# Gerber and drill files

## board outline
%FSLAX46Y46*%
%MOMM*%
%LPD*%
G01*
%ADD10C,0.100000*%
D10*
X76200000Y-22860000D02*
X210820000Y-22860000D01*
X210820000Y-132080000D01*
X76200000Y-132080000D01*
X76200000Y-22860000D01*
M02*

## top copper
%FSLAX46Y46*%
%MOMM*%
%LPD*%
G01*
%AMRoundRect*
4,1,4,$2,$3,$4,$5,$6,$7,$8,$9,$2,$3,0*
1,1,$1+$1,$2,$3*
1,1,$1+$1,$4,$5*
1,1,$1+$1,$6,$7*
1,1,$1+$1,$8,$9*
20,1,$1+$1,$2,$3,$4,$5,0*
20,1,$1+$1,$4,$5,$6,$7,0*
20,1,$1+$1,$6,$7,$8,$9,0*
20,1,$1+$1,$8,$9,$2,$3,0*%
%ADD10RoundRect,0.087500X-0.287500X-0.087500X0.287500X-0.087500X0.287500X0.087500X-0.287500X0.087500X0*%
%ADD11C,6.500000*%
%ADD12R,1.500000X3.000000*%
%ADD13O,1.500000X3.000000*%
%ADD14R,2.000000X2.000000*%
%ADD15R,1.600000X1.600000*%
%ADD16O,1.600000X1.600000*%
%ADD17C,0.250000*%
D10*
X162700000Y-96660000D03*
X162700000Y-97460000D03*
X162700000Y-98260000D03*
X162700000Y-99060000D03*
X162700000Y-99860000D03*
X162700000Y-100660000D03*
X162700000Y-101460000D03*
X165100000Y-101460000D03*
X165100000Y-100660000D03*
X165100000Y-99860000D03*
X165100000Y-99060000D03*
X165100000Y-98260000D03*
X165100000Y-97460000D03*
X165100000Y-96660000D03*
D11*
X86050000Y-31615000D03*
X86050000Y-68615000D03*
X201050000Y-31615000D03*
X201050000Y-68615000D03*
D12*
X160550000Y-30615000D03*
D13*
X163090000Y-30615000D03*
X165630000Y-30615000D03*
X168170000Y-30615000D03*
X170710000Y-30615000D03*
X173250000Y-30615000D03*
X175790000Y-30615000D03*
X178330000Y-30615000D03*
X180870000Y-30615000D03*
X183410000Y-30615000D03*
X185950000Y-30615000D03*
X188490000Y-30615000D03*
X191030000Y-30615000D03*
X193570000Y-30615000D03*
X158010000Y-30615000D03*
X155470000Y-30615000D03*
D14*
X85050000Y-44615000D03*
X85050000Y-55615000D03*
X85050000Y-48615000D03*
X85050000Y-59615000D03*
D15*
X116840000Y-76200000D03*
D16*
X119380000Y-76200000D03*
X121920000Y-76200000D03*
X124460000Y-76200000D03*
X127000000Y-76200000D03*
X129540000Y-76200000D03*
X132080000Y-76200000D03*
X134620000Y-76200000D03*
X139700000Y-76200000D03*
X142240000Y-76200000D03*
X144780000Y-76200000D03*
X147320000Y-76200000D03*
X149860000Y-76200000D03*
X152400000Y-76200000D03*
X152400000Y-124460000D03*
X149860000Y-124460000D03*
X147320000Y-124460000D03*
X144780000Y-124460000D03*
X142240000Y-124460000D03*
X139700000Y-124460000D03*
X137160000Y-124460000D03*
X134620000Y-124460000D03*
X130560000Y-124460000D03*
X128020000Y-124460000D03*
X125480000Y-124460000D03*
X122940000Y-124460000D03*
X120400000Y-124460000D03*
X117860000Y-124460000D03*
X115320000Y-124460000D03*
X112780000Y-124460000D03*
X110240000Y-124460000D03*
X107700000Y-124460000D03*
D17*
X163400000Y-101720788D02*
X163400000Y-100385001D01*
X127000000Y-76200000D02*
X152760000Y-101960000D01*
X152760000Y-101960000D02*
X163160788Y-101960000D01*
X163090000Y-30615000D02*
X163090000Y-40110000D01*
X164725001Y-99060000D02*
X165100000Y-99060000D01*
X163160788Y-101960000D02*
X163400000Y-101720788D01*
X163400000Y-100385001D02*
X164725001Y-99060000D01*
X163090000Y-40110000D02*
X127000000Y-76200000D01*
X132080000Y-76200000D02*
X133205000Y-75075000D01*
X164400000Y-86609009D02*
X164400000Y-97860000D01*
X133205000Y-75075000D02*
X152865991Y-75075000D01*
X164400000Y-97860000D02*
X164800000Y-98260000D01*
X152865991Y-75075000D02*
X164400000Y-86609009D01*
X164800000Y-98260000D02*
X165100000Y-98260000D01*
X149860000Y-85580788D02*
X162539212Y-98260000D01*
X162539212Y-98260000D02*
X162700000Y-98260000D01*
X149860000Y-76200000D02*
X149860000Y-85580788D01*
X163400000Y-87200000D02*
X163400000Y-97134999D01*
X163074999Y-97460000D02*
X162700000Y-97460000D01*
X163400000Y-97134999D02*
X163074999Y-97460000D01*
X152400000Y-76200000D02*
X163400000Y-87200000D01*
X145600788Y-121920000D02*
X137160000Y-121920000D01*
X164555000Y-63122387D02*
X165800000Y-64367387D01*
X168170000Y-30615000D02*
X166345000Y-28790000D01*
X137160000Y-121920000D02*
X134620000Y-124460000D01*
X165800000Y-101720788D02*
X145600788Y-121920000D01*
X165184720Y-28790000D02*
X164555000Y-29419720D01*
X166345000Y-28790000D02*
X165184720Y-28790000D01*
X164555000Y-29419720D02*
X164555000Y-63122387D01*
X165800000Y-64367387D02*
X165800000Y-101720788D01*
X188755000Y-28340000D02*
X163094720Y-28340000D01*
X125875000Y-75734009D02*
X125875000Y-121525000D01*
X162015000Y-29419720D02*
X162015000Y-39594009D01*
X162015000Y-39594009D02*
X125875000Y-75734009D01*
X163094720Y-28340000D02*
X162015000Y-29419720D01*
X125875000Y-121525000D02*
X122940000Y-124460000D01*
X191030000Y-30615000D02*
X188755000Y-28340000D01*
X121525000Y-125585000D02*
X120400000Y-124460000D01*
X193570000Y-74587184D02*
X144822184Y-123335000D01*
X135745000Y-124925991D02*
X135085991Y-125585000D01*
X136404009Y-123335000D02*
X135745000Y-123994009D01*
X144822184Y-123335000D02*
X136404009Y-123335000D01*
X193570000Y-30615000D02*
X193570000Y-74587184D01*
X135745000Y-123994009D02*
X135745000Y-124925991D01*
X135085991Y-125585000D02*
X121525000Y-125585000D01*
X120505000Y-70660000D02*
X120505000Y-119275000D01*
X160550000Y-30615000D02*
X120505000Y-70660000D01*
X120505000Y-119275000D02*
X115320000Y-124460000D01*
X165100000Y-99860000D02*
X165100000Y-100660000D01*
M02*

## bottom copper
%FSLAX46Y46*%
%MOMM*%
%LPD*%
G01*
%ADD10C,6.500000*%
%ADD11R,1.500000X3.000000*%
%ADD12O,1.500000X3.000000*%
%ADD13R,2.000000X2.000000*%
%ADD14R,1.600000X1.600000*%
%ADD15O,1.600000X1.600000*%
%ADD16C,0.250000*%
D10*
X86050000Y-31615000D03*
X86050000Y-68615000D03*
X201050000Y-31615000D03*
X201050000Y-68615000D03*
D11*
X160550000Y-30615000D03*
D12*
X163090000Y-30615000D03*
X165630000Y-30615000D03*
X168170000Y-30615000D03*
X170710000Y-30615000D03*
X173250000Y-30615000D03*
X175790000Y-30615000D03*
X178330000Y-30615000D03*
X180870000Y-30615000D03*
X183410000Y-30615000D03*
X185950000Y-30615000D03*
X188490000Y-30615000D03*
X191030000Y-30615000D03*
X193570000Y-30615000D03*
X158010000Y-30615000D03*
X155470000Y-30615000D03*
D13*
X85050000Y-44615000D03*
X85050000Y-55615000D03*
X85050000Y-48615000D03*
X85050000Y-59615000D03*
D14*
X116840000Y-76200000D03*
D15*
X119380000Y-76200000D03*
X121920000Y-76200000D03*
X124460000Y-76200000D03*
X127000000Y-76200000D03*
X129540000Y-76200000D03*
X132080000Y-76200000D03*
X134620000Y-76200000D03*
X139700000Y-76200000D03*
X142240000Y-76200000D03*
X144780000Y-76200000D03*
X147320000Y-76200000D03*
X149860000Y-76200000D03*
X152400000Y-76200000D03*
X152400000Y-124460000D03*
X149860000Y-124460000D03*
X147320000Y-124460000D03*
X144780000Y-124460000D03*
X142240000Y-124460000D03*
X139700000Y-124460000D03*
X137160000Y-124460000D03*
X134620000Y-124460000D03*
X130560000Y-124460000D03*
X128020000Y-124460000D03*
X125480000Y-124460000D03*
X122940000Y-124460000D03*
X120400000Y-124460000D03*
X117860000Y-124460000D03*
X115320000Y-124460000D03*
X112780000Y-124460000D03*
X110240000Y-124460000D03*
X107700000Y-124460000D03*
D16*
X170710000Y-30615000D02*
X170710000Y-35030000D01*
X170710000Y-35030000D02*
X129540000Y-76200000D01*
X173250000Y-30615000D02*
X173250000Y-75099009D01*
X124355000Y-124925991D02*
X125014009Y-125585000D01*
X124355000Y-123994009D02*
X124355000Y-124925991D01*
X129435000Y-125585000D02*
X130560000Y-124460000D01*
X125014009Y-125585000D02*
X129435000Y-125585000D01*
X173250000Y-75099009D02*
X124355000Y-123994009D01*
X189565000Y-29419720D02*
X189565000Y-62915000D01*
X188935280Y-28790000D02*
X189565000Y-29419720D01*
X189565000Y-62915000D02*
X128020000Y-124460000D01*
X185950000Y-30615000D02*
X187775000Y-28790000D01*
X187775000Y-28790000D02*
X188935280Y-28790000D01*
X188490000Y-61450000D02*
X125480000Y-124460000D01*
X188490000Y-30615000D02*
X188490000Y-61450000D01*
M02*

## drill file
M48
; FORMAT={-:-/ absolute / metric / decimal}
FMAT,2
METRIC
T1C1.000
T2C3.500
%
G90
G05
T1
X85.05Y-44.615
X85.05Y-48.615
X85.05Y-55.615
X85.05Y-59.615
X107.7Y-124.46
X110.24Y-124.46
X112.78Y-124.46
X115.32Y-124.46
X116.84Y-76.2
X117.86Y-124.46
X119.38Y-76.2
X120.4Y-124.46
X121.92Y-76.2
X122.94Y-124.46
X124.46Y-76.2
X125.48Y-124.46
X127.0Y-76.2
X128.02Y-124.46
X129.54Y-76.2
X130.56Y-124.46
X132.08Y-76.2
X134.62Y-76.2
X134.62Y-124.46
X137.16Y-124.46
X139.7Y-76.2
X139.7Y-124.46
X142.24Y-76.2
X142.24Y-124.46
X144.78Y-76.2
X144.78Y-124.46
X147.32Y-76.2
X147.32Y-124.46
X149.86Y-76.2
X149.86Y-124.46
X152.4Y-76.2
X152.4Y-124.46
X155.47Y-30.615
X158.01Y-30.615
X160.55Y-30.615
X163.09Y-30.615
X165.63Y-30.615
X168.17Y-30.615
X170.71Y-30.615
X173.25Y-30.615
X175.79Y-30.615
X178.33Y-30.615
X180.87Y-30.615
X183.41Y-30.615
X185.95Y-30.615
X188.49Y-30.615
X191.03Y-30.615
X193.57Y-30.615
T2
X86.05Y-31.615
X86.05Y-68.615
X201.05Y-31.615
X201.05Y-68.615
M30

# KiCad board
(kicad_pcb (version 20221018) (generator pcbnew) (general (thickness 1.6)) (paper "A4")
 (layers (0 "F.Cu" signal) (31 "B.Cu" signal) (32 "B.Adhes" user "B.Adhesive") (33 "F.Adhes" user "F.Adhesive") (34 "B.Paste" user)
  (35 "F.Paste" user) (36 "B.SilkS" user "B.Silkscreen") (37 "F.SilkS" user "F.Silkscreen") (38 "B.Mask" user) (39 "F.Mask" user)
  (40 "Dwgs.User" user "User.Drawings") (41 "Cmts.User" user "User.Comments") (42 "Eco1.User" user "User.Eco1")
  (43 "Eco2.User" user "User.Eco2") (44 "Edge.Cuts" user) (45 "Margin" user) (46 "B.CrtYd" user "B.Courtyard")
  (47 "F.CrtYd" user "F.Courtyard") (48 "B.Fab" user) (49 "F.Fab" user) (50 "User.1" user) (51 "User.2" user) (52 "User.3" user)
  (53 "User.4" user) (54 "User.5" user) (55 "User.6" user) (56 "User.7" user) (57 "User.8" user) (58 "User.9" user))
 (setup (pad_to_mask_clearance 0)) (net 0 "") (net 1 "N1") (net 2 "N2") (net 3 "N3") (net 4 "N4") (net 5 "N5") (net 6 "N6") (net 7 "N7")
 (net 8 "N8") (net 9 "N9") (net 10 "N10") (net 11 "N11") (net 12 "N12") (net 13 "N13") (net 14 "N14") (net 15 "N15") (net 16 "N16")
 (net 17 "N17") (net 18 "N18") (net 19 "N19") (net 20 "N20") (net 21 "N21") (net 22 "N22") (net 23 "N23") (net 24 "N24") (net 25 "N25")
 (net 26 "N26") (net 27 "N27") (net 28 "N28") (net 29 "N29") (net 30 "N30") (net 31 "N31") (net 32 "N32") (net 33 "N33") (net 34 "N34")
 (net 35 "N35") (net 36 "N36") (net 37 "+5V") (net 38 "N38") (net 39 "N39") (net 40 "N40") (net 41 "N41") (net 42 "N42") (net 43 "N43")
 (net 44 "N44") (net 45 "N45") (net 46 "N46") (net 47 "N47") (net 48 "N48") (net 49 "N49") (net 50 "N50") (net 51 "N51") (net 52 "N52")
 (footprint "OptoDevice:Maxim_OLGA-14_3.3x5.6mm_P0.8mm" (layer "F.Cu") (at 163.9 99.06)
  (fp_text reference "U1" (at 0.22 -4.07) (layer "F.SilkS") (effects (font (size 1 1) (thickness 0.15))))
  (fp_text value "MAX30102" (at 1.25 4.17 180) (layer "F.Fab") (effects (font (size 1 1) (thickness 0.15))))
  (pad "1" smd roundrect (at -1.2 -2.4) (size 0.75 0.35) (layers "F.Cu" "F.Paste" "F.Mask") (roundrect_rratio 0.25) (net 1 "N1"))
  (pad "2" smd roundrect (at -1.2 -1.6) (size 0.75 0.35) (layers "F.Cu" "F.Paste" "F.Mask") (roundrect_rratio 0.25) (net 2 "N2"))
  (pad "3" smd roundrect (at -1.2 -0.8) (size 0.75 0.35) (layers "F.Cu" "F.Paste" "F.Mask") (roundrect_rratio 0.25) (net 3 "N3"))
  (pad "4" smd roundrect (at -1.2 0) (size 0.75 0.35) (layers "F.Cu" "F.Paste" "F.Mask") (roundrect_rratio 0.25) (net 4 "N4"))
  (pad "5" smd roundrect (at -1.2 0.8) (size 0.75 0.35) (layers "F.Cu" "F.Paste" "F.Mask") (roundrect_rratio 0.25) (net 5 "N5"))
  (pad "6" smd roundrect (at -1.2 1.6) (size 0.75 0.35) (layers "F.Cu" "F.Paste" "F.Mask") (roundrect_rratio 0.25) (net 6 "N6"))
  (pad "7" smd roundrect (at -1.2 2.4) (size 0.75 0.35) (layers "F.Cu" "F.Paste" "F.Mask") (roundrect_rratio 0.25) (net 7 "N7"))
  (pad "8" smd roundrect (at 1.2 2.4) (size 0.75 0.35) (layers "F.Cu" "F.Paste" "F.Mask") (roundrect_rratio 0.25) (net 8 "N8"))
  (pad "9" smd roundrect (at 1.2 1.6) (size 0.75 0.35) (layers "F.Cu" "F.Paste" "F.Mask") (roundrect_rratio 0.25) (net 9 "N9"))
  (pad "10" smd roundrect (at 1.2 0.8) (size 0.75 0.35) (layers "F.Cu" "F.Paste" "F.Mask") (roundrect_rratio 0.25) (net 9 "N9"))
  (pad "11" smd roundrect (at 1.2 0) (size 0.75 0.35) (layers "F.Cu" "F.Paste" "F.Mask") (roundrect_rratio 0.25) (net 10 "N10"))
  (pad "12" smd roundrect (at 1.2 -0.8) (size 0.75 0.35) (layers "F.Cu" "F.Paste" "F.Mask") (roundrect_rratio 0.25) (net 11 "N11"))
  (pad "13" smd roundrect (at 1.2 -1.6) (size 0.75 0.35) (layers "F.Cu" "F.Paste" "F.Mask") (roundrect_rratio 0.25) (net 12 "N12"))
  (pad "14" smd roundrect (at 1.2 -2.4) (size 0.75 0.35) (layers "F.Cu" "F.Paste" "F.Mask") (roundrect_rratio 0.25) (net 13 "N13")))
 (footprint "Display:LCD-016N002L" (layer "F.Cu") (at 160.55 30.615)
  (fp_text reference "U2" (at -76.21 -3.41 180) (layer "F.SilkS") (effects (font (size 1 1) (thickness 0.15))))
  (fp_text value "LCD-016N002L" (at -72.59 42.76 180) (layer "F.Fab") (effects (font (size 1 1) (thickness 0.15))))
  (pad "" thru_hole circle (at -74.5 1 180) (size 6.5 6.5) (drill 3.5) (layers "*.Cu" "*.Mask"))
  (pad "" thru_hole circle (at -74.5 38 180) (size 6.5 6.5) (drill 3.5) (layers "*.Cu" "*.Mask"))
  (pad "" thru_hole circle (at 40.5 1 180) (size 6.5 6.5) (drill 3.5) (layers "*.Cu" "*.Mask"))
  (pad "" thru_hole circle (at 40.5 38 180) (size 6.5 6.5) (drill 3.5) (layers "*.Cu" "*.Mask"))
  (pad "1" thru_hole rect (at 0 0 180) (size 1.5 3) (drill 1) (layers "*.Cu" "*.Mask") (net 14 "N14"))
  (pad "2" thru_hole oval (at 2.54 0 180) (size 1.5 3) (drill 1) (layers "*.Cu" "*.Mask") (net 10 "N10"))
  (pad "3" thru_hole oval (at 5.08 0 180) (size 1.5 3) (drill 1) (layers "*.Cu" "*.Mask") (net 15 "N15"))
  (pad "4" thru_hole oval (at 7.62 0 180) (size 1.5 3) (drill 1) (layers "*.Cu" "*.Mask") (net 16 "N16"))
  (pad "5" thru_hole oval (at 10.16 0 180) (size 1.5 3) (drill 1) (layers "*.Cu" "*.Mask") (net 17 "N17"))
  (pad "6" thru_hole oval (at 12.7 0 180) (size 1.5 3) (drill 1) (layers "*.Cu" "*.Mask") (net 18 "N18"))
  (pad "7" thru_hole oval (at 15.24 0 180) (size 1.5 3) (drill 1) (layers "*.Cu" "*.Mask") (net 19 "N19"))
  (pad "8" thru_hole oval (at 17.78 0 180) (size 1.5 3) (drill 1) (layers "*.Cu" "*.Mask") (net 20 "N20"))
  (pad "9" thru_hole oval (at 20.32 0 180) (size 1.5 3) (drill 1) (layers "*.Cu" "*.Mask") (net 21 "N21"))
  (pad "10" thru_hole oval (at 22.86 0 180) (size 1.5 3) (drill 1) (layers "*.Cu" "*.Mask") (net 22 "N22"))
  (pad "11" thru_hole oval (at 25.4 0 180) (size 1.5 3) (drill 1) (layers "*.Cu" "*.Mask") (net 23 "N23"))
  (pad "12" thru_hole oval (at 27.94 0 180) (size 1.5 3) (drill 1) (layers "*.Cu" "*.Mask") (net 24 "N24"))
  (pad "13" thru_hole oval (at 30.48 0 180) (size 1.5 3) (drill 1) (layers "*.Cu" "*.Mask") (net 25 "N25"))
  (pad "14" thru_hole oval (at 33.02 0 180) (size 1.5 3) (drill 1) (layers "*.Cu" "*.Mask") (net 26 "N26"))
  (pad "15" thru_hole oval (at -2.54 0 180) (size 1.5 3) (drill 1) (layers "*.Cu" "*.Mask") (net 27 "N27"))
  (pad "16" thru_hole oval (at -5.08 0 180) (size 1.5 3) (drill 1) (layers "*.Cu" "*.Mask") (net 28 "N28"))
  (pad "A1" thru_hole rect (at -75.5 14 180) (size 2 2) (drill 1) (layers "*.Cu" "*.Mask") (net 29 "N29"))
  (pad "A2" thru_hole rect (at -75.5 25 180) (size 2 2) (drill 1) (layers "*.Cu" "*.Mask") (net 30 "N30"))
  (pad "K1" thru_hole rect (at -75.5 18 180) (size 2 2) (drill 1) (layers "*.Cu" "*.Mask") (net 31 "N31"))
  (pad "K2" thru_hole rect (at -75.5 29 180) (size 2 2) (drill 1) (layers "*.Cu" "*.Mask") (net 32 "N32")))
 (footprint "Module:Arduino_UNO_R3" (layer "F.Cu") (at 116.84 76.2)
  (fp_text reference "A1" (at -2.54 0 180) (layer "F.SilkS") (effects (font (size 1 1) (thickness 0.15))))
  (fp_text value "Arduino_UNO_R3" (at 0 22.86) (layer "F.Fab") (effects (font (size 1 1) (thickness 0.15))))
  (pad "1" thru_hole rect (at 0 0 90) (size 1.6 1.6) (drill 1) (layers "*.Cu" "*.Mask") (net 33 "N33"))
  (pad "2" thru_hole oval (at 2.54 0 90) (size 1.6 1.6) (drill 1) (layers "*.Cu" "*.Mask") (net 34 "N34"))
  (pad "3" thru_hole oval (at 5.08 0 90) (size 1.6 1.6) (drill 1) (layers "*.Cu" "*.Mask") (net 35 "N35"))
  (pad "4" thru_hole oval (at 7.62 0 90) (size 1.6 1.6) (drill 1) (layers "*.Cu" "*.Mask") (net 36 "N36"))
  (pad "5" thru_hole oval (at 10.16 0 90) (size 1.6 1.6) (drill 1) (layers "*.Cu" "*.Mask") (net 10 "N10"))
  (pad "6" thru_hole oval (at 12.7 0 90) (size 1.6 1.6) (drill 1) (layers "*.Cu" "*.Mask") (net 17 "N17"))
  (pad "7" thru_hole oval (at 15.24 0 90) (size 1.6 1.6) (drill 1) (layers "*.Cu" "*.Mask") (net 11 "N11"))
  (pad "8" thru_hole oval (at 17.78 0 90) (size 1.6 1.6) (drill 1) (layers "*.Cu" "*.Mask") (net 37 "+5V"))
  (pad "9" thru_hole oval (at 22.86 0 90) (size 1.6 1.6) (drill 1) (layers "*.Cu" "*.Mask") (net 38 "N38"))
  (pad "10" thru_hole oval (at 25.4 0 90) (size 1.6 1.6) (drill 1) (layers "*.Cu" "*.Mask") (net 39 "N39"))
  (pad "11" thru_hole oval (at 27.94 0 90) (size 1.6 1.6) (drill 1) (layers "*.Cu" "*.Mask") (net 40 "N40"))
  (pad "12" thru_hole oval (at 30.48 0 90) (size 1.6 1.6) (drill 1) (layers "*.Cu" "*.Mask") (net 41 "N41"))
  (pad "13" thru_hole oval (at 33.02 0 90) (size 1.6 1.6) (drill 1) (layers "*.Cu" "*.Mask") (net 3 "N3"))
  (pad "14" thru_hole oval (at 35.56 0 90) (size 1.6 1.6) (drill 1) (layers "*.Cu" "*.Mask") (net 2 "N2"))
  (pad "15" thru_hole oval (at 35.56 48.26 90) (size 1.6 1.6) (drill 1) (layers "*.Cu" "*.Mask") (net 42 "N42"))
  (pad "16" thru_hole oval (at 33.02 48.26 90) (size 1.6 1.6) (drill 1) (layers "*.Cu" "*.Mask") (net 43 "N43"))
  (pad "17" thru_hole oval (at 30.48 48.26 90) (size 1.6 1.6) (drill 1) (layers "*.Cu" "*.Mask") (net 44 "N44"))
  (pad "18" thru_hole oval (at 27.94 48.26 90) (size 1.6 1.6) (drill 1) (layers "*.Cu" "*.Mask") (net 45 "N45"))
  (pad "19" thru_hole oval (at 25.4 48.26 90) (size 1.6 1.6) (drill 1) (layers "*.Cu" "*.Mask") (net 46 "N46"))
  (pad "20" thru_hole oval (at 22.86 48.26 90) (size 1.6 1.6) (drill 1) (layers "*.Cu" "*.Mask") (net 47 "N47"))
  (pad "21" thru_hole oval (at 20.32 48.26 90) (size 1.6 1.6) (drill 1) (layers "*.Cu" "*.Mask") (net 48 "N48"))
  (pad "22" thru_hole oval (at 17.78 48.26 90) (size 1.6 1.6) (drill 1) (layers "*.Cu" "*.Mask") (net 16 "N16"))
  (pad "23" thru_hole oval (at 13.72 48.26 90) (size 1.6 1.6) (drill 1) (layers "*.Cu" "*.Mask") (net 18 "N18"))
  (pad "24" thru_hole oval (at 11.18 48.26 90) (size 1.6 1.6) (drill 1) (layers "*.Cu" "*.Mask") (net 23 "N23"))
  (pad "25" thru_hole oval (at 8.64 48.26 90) (size 1.6 1.6) (drill 1) (layers "*.Cu" "*.Mask") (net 24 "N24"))
  (pad "26" thru_hole oval (at 6.1 48.26 90) (size 1.6 1.6) (drill 1) (layers "*.Cu" "*.Mask") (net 25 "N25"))
  (pad "27" thru_hole oval (at 3.56 48.26 90) (size 1.6 1.6) (drill 1) (layers "*.Cu" "*.Mask") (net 26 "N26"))
  (pad "28" thru_hole oval (at 1.02 48.26 90) (size 1.6 1.6) (drill 1) (layers "*.Cu" "*.Mask") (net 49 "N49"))
  (pad "29" thru_hole oval (at -1.52 48.26 90) (size 1.6 1.6) (drill 1) (layers "*.Cu" "*.Mask") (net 14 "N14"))
  (pad "30" thru_hole oval (at -4.06 48.26 90) (size 1.6 1.6) (drill 1) (layers "*.Cu" "*.Mask") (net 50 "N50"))
  (pad "31" thru_hole oval (at -6.6 48.26 90) (size 1.6 1.6) (drill 1) (layers "*.Cu" "*.Mask") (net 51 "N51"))
  (pad "32" thru_hole oval (at -9.14 48.26 90) (size 1.6 1.6) (drill 1) (layers "*.Cu" "*.Mask") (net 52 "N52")))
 (gr_rect (start 76.2 22.86) (end 210.82 132.08) (stroke (width 0.1) (type default)) (fill none) (layer "Edge.Cuts"))
 (segment (start 163.4 101.720788) (end 163.4 100.385001) (width 0.25) (layer "F.Cu") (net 10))
 (segment (start 127 76.2) (end 152.76 101.96) (width 0.25) (layer "F.Cu") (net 10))
 (segment (start 152.76 101.96) (end 163.160788 101.96) (width 0.25) (layer "F.Cu") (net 10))
 (segment (start 163.09 30.615) (end 163.09 40.11) (width 0.25) (layer "F.Cu") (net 10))
 (segment (start 164.725001 99.06) (end 165.1 99.06) (width 0.25) (layer "F.Cu") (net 10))
 (segment (start 163.160788 101.96) (end 163.4 101.720788) (width 0.25) (layer "F.Cu") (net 10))
 (segment (start 163.4 100.385001) (end 164.725001 99.06) (width 0.25) (layer "F.Cu") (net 10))
 (segment (start 163.09 40.11) (end 127 76.2) (width 0.25) (layer "F.Cu") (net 10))
 (segment (start 170.71 30.615) (end 170.71 35.03) (width 0.25) (layer "B.Cu") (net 17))
 (segment (start 170.71 35.03) (end 129.54 76.2) (width 0.25) (layer "B.Cu") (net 17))
 (segment (start 132.08 76.2) (end 133.205 75.075) (width 0.25) (layer "F.Cu") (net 11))
 (segment (start 164.4 86.609009) (end 164.4 97.86) (width 0.25) (layer "F.Cu") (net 11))
 (segment (start 133.205 75.075) (end 152.865991 75.075) (width 0.25) (layer "F.Cu") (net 11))
 (segment (start 164.4 97.86) (end 164.8 98.26) (width 0.25) (layer "F.Cu") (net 11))
 (segment (start 152.865991 75.075) (end 164.4 86.609009) (width 0.25) (layer "F.Cu") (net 11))
 (segment (start 164.8 98.26) (end 165.1 98.26) (width 0.25) (layer "F.Cu") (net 11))
 (segment (start 149.86 85.580788) (end 162.539212 98.26) (width 0.25) (layer "F.Cu") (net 3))
 (segment (start 162.539212 98.26) (end 162.7 98.26) (width 0.25) (layer "F.Cu") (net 3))
 (segment (start 149.86 76.2) (end 149.86 85.580788) (width 0.25) (layer "F.Cu") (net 3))
 (segment (start 163.4 87.2) (end 163.4 97.134999) (width 0.25) (layer "F.Cu") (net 2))
 (segment (start 163.074999 97.46) (end 162.7 97.46) (width 0.25) (layer "F.Cu") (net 2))
 (segment (start 163.4 97.134999) (end 163.074999 97.46) (width 0.25) (layer "F.Cu") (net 2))
 (segment (start 152.4 76.2) (end 163.4 87.2) (width 0.25) (layer "F.Cu") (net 2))
 (segment (start 145.600788 121.92) (end 137.16 121.92) (width 0.25) (layer "F.Cu") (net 16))
 (segment (start 164.555 63.122387) (end 165.8 64.367387) (width 0.25) (layer "F.Cu") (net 16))
 (segment (start 168.17 30.615) (end 166.345 28.79) (width 0.25) (layer "F.Cu") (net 16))
 (segment (start 137.16 121.92) (end 134.62 124.46) (width 0.25) (layer "F.Cu") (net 16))
 (segment (start 165.8 101.720788) (end 145.600788 121.92) (width 0.25) (layer "F.Cu") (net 16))
 (segment (start 165.18472 28.79) (end 164.555 29.41972) (width 0.25) (layer "F.Cu") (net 16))
 (segment (start 166.345 28.79) (end 165.18472 28.79) (width 0.25) (layer "F.Cu") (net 16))
 (segment (start 164.555 29.41972) (end 164.555 63.122387) (width 0.25) (layer "F.Cu") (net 16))
 (segment (start 165.8 64.367387) (end 165.8 101.720788) (width 0.25) (layer "F.Cu") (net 16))
 (segment (start 173.25 30.615) (end 173.25 75.099009) (width 0.25) (layer "B.Cu") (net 18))
 (segment (start 124.355 124.925991) (end 125.014009 125.585) (width 0.25) (layer "B.Cu") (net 18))
 (segment (start 124.355 123.994009) (end 124.355 124.925991) (width 0.25) (layer "B.Cu") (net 18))
 (segment (start 129.435 125.585) (end 130.56 124.46) (width 0.25) (layer "B.Cu") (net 18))
 (segment (start 125.014009 125.585) (end 129.435 125.585) (width 0.25) (layer "B.Cu") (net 18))
 (segment (start 173.25 75.099009) (end 124.355 123.994009) (width 0.25) (layer "B.Cu") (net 18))
 (segment (start 189.565 29.41972) (end 189.565 62.915) (width 0.25) (layer "B.Cu") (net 23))
 (segment (start 188.93528 28.79) (end 189.565 29.41972) (width 0.25) (layer "B.Cu") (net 23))
 (segment (start 189.565 62.915) (end 128.02 124.46) (width 0.25) (layer "B.Cu") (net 23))
 (segment (start 185.95 30.615) (end 187.775 28.79) (width 0.25) (layer "B.Cu") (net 23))
 (segment (start 187.775 28.79) (end 188.93528 28.79) (width 0.25) (layer "B.Cu") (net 23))
 (segment (start 188.49 61.45) (end 125.48 124.46) (width 0.25) (layer "B.Cu") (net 24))
 (segment (start 188.49 30.615) (end 188.49 61.45) (width 0.25) (layer "B.Cu") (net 24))
 (segment (start 188.755 28.34) (end 163.09472 28.34) (width 0.25) (layer "F.Cu") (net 25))
 (segment (start 125.875 75.734009) (end 125.875 121.525) (width 0.25) (layer "F.Cu") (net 25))
 (segment (start 162.015 29.41972) (end 162.015 39.594009) (width 0.25) (layer "F.Cu") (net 25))
 (segment (start 162.015 39.594009) (end 125.875 75.734009) (width 0.25) (layer "F.Cu") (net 25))
 (segment (start 163.09472 28.34) (end 162.015 29.41972) (width 0.25) (layer "F.Cu") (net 25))
 (segment (start 125.875 121.525) (end 122.94 124.46) (width 0.25) (layer "F.Cu") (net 25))
 (segment (start 191.03 30.615) (end 188.755 28.34) (width 0.25) (layer "F.Cu") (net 25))
 (segment (start 121.525 125.585) (end 120.4 124.46) (width 0.25) (layer "F.Cu") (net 26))
 (segment (start 193.57 74.587184) (end 144.822184 123.335) (width 0.25) (layer "F.Cu") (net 26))
 (segment (start 135.745 124.925991) (end 135.085991 125.585) (width 0.25) (layer "F.Cu") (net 26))
 (segment (start 136.404009 123.335) (end 135.745 123.994009) (width 0.25) (layer "F.Cu") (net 26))
 (segment (start 144.822184 123.335) (end 136.404009 123.335) (width 0.25) (layer "F.Cu") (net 26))
 (segment (start 193.57 30.615) (end 193.57 74.587184) (width 0.25) (layer "F.Cu") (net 26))
 (segment (start 135.745 123.994009) (end 135.745 124.925991) (width 0.25) (layer "F.Cu") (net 26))
 (segment (start 135.085991 125.585) (end 121.525 125.585) (width 0.25) (layer "F.Cu") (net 26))
 (segment (start 120.505 70.66) (end 120.505 119.275) (width 0.25) (layer "F.Cu") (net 14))
 (segment (start 160.55 30.615) (end 120.505 70.66) (width 0.25) (layer "F.Cu") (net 14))
 (segment (start 120.505 119.275) (end 115.32 124.46) (width 0.25) (layer "F.Cu") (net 14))
 (segment (start 165.1 99.86) (end 165.1 100.66) (width 0.25) (layer "F.Cu") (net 9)))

